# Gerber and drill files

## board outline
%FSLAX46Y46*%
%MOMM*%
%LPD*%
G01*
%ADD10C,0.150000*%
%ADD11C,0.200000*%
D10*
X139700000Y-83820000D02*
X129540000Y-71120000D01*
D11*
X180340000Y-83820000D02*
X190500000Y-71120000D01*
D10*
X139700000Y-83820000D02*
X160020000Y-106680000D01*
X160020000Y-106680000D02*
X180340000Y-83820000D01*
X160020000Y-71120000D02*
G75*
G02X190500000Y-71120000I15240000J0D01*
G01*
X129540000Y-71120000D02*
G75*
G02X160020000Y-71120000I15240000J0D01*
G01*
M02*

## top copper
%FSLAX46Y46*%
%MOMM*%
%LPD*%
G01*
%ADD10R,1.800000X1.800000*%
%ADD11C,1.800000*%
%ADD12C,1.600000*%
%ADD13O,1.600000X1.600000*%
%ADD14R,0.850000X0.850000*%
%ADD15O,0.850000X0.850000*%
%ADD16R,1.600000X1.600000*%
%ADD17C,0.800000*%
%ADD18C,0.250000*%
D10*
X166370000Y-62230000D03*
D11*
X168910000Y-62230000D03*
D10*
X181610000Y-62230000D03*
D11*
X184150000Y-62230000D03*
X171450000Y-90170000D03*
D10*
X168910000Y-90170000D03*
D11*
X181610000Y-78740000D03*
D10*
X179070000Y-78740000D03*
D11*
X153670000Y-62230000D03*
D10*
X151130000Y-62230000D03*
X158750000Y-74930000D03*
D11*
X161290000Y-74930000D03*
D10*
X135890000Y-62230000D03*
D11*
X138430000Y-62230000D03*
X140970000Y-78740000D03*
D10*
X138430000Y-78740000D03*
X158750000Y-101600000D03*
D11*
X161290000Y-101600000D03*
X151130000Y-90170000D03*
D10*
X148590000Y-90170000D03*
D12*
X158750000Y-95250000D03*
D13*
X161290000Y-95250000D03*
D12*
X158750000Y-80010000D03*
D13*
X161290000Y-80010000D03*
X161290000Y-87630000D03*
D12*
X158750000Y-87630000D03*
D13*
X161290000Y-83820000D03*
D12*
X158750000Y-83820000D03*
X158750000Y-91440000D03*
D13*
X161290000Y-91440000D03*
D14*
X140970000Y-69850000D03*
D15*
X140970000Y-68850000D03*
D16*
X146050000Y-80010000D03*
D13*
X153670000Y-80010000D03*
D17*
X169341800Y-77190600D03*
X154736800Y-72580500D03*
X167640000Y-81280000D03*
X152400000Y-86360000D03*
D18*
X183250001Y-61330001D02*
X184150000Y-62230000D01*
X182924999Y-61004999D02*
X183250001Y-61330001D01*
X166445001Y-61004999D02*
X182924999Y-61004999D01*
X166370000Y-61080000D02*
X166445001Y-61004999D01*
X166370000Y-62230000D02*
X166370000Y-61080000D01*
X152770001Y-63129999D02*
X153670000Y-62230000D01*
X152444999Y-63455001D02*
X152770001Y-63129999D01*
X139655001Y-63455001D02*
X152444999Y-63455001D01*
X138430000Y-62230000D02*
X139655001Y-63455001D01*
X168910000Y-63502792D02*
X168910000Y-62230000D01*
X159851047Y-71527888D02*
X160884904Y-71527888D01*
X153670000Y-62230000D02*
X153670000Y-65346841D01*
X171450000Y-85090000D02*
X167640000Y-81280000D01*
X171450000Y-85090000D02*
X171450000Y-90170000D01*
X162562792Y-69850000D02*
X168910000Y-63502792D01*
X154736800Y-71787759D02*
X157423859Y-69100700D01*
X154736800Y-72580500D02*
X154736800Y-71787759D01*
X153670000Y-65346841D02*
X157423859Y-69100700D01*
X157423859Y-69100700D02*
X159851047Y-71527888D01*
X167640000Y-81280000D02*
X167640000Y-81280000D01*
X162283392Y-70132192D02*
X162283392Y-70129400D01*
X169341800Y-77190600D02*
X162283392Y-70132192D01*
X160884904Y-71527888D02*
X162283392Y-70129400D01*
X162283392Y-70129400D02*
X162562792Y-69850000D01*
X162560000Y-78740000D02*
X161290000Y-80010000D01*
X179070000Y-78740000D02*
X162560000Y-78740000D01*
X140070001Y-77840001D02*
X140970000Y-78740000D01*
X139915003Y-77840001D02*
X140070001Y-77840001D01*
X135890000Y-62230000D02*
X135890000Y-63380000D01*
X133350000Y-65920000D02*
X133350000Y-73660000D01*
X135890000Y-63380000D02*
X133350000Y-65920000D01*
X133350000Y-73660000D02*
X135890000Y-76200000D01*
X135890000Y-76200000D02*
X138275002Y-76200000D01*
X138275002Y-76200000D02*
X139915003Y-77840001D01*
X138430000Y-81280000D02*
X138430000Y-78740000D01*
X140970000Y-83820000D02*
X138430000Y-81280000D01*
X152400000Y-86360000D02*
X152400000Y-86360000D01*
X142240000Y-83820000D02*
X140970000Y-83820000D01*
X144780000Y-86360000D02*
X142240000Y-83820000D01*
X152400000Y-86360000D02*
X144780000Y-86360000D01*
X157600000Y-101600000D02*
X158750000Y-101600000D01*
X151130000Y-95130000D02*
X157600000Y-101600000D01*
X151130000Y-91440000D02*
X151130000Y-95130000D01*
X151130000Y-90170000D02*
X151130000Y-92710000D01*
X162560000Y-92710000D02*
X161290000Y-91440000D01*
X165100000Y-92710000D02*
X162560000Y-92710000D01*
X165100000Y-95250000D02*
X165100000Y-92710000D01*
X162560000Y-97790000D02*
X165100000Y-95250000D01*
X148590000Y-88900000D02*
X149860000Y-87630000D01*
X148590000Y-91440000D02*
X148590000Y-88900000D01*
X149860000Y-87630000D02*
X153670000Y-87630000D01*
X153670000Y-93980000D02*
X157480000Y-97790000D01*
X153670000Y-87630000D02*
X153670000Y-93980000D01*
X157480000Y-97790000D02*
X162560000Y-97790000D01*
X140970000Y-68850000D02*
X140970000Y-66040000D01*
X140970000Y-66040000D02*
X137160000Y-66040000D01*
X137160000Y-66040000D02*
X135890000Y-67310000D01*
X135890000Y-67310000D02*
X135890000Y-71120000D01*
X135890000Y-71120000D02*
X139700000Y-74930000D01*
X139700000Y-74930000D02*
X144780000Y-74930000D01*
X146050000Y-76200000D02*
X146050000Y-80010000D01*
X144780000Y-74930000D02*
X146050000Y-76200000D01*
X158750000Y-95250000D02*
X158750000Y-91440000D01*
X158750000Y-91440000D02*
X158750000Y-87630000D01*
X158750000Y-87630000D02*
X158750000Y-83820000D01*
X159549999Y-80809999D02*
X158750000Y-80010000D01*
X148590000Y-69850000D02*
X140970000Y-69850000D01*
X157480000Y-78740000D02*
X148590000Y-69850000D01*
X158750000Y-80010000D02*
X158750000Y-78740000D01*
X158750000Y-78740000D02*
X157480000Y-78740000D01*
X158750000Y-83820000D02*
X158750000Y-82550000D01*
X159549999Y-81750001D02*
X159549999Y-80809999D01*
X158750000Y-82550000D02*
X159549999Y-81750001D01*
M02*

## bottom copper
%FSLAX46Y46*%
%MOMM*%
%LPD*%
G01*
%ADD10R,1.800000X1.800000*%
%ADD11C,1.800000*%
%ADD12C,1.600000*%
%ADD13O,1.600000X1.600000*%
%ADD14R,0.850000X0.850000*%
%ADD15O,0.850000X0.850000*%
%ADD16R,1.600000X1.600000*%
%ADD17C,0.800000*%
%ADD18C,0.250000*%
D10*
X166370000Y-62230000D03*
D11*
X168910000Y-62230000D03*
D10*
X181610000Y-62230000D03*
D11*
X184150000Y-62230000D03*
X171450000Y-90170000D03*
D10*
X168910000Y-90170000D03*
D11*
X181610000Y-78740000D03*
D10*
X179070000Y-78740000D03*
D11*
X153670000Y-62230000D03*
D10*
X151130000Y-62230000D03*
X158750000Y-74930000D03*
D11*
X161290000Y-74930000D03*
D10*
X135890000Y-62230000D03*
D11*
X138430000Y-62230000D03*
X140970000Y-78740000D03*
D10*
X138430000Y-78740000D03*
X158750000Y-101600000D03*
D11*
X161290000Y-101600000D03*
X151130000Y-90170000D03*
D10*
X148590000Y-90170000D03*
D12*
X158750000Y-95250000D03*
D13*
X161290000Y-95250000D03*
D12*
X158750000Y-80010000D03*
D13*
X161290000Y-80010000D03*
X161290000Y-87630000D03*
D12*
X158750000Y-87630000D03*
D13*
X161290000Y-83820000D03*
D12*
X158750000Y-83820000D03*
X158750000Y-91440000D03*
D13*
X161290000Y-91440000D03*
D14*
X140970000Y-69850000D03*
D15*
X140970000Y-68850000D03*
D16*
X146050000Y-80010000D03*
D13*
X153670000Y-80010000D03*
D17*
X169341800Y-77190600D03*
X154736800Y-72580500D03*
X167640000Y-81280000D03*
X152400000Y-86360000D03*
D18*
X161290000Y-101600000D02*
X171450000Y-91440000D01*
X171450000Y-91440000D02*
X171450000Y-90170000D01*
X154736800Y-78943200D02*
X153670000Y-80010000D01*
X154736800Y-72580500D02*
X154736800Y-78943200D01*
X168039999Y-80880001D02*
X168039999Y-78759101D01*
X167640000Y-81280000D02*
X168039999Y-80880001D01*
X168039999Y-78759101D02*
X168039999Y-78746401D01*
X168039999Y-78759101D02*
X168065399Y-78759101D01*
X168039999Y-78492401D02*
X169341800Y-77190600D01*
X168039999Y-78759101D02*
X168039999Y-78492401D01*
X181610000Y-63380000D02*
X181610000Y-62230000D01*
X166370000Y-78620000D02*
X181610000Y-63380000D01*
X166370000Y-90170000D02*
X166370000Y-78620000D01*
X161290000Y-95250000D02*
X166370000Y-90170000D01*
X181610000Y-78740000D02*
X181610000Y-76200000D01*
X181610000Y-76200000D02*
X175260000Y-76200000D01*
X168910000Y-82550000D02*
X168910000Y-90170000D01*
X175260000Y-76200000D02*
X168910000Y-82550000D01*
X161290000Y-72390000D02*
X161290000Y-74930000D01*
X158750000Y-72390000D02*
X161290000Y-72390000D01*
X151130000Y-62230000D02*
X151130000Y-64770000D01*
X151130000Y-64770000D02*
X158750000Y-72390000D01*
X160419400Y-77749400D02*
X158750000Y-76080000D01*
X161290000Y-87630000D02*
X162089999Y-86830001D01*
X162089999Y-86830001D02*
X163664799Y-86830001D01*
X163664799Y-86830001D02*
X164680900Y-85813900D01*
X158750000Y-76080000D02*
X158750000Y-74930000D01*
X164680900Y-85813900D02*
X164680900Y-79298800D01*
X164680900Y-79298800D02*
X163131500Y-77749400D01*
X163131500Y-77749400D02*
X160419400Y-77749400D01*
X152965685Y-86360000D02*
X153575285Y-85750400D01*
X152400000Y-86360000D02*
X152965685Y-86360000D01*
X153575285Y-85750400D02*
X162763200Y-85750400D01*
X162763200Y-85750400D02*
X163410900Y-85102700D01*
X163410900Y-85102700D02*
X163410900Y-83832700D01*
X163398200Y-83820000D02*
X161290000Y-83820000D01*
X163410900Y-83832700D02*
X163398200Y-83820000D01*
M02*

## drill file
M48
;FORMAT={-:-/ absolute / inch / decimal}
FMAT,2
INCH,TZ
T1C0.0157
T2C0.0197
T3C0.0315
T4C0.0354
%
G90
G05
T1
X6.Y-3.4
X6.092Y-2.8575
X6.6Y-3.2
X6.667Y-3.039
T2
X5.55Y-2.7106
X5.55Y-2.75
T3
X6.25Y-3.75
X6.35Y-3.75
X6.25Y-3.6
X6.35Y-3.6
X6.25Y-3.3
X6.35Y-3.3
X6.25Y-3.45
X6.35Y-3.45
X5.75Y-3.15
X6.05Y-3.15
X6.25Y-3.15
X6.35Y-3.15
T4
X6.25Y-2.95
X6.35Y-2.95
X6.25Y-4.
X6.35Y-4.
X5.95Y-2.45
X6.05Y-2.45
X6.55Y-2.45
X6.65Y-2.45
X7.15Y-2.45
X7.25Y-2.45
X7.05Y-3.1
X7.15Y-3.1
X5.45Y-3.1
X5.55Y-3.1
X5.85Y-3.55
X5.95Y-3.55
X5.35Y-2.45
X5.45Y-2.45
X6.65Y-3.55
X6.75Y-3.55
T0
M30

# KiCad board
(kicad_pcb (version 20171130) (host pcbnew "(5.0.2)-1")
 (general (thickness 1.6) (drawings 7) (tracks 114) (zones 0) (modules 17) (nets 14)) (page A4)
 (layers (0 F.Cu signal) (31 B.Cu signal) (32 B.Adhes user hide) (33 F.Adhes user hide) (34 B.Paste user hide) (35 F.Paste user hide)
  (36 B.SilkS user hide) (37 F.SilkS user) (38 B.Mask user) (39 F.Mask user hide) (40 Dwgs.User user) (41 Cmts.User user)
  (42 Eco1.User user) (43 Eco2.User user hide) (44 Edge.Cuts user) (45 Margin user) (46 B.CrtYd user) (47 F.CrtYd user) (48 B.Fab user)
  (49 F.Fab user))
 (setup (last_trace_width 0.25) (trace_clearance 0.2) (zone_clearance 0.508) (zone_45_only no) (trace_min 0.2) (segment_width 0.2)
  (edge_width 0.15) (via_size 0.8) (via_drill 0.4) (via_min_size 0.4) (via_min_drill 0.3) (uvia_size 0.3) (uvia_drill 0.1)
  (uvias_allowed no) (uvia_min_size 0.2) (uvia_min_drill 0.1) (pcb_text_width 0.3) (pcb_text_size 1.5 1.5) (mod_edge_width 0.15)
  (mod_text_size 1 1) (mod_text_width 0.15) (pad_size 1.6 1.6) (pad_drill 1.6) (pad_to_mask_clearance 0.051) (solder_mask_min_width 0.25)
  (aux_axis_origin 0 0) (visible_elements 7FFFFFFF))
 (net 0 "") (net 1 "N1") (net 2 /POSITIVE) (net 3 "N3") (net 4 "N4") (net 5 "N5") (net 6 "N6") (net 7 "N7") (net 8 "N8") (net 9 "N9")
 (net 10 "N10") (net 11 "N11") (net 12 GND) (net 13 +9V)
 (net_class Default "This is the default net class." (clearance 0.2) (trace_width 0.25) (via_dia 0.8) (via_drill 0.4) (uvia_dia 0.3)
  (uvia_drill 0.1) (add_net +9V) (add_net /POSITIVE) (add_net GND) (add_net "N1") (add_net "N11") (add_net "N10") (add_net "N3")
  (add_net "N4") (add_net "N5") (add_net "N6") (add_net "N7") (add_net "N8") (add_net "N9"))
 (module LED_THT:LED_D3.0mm (layer F.Cu) (at 166.37 62.23)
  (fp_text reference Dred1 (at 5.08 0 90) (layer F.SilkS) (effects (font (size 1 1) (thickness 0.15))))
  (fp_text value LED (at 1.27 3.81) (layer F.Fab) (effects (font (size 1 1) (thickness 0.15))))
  (pad 1 thru_hole rect (at 0 0) (size 1.8 1.8) (drill 0.9) (layers *.Cu *.Mask) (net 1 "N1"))
  (pad 2 thru_hole circle (at 2.54 0) (size 1.8 1.8) (drill 0.9) (layers *.Cu *.Mask) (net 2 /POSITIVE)))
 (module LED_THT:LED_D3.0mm (layer F.Cu) (at 181.61 62.23)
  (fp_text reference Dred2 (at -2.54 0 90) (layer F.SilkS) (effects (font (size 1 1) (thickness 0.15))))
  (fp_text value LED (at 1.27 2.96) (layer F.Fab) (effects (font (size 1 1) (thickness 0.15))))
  (pad 1 thru_hole rect (at 0 0) (size 1.8 1.8) (drill 0.9) (layers *.Cu *.Mask) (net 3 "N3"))
  (pad 2 thru_hole circle (at 2.54 0) (size 1.8 1.8) (drill 0.9) (layers *.Cu *.Mask) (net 1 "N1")))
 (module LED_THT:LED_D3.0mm (layer F.Cu) (at 168.91 90.17)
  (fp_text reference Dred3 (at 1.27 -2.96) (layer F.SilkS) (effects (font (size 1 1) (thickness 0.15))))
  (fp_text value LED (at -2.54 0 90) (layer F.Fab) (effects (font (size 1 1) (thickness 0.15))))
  (pad 2 thru_hole circle (at 2.54 0) (size 1.8 1.8) (drill 0.9) (layers *.Cu *.Mask) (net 2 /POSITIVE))
  (pad 1 thru_hole rect (at 0 0) (size 1.8 1.8) (drill 0.9) (layers *.Cu *.Mask) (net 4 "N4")))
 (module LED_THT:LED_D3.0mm (layer F.Cu) (at 179.07 78.74)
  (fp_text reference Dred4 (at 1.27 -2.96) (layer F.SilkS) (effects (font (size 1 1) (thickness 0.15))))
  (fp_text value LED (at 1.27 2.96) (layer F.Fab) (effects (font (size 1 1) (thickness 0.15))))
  (pad 2 thru_hole circle (at 2.54 0) (size 1.8 1.8) (drill 0.9) (layers *.Cu *.Mask) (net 4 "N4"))
  (pad 1 thru_hole rect (at 0 0) (size 1.8 1.8) (drill 0.9) (layers *.Cu *.Mask) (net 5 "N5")))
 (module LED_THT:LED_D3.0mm (layer F.Cu) (at 151.13 62.23)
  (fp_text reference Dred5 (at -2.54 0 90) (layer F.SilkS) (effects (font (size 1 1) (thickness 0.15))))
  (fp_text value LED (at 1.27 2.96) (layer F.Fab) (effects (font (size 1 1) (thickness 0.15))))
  (pad 2 thru_hole circle (at 2.54 0) (size 1.8 1.8) (drill 0.9) (layers *.Cu *.Mask) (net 2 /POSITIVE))
  (pad 1 thru_hole rect (at 0 0) (size 1.8 1.8) (drill 0.9) (layers *.Cu *.Mask) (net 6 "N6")))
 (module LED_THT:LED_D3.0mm (layer F.Cu) (at 158.75 74.93)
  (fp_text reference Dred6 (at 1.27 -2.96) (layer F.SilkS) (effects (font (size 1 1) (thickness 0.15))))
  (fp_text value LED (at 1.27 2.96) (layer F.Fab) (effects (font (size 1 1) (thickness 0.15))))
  (pad 1 thru_hole rect (at 0 0) (size 1.8 1.8) (drill 0.9) (layers *.Cu *.Mask) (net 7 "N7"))
  (pad 2 thru_hole circle (at 2.54 0) (size 1.8 1.8) (drill 0.9) (layers *.Cu *.Mask) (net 6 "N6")))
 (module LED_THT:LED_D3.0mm (layer F.Cu) (at 135.89 62.23)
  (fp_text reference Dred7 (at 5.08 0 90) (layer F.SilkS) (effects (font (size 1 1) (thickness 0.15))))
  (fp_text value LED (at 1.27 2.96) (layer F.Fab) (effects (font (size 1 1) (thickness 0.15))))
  (pad 1 thru_hole rect (at 0 0) (size 1.8 1.8) (drill 0.9) (layers *.Cu *.Mask) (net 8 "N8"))
  (pad 2 thru_hole circle (at 2.54 0) (size 1.8 1.8) (drill 0.9) (layers *.Cu *.Mask) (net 2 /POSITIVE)))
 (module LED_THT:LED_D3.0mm (layer F.Cu) (at 138.43 78.74)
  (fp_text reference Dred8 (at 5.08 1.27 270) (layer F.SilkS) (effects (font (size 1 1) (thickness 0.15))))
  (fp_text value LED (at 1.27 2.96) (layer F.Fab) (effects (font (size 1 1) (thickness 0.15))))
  (pad 2 thru_hole circle (at 2.54 0) (size 1.8 1.8) (drill 0.9) (layers *.Cu *.Mask) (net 8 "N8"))
  (pad 1 thru_hole rect (at 0 0) (size 1.8 1.8) (drill 0.9) (layers *.Cu *.Mask) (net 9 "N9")))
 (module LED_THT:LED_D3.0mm (layer F.Cu) (at 158.75 101.6)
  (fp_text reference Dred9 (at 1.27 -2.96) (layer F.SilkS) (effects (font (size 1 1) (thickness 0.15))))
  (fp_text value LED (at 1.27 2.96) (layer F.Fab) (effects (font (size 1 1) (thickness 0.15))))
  (pad 1 thru_hole rect (at 0 0) (size 1.8 1.8) (drill 0.9) (layers *.Cu *.Mask) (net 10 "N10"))
  (pad 2 thru_hole circle (at 2.54 0) (size 1.8 1.8) (drill 0.9) (layers *.Cu *.Mask) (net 2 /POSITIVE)))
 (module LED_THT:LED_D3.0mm (layer F.Cu) (at 148.59 90.17)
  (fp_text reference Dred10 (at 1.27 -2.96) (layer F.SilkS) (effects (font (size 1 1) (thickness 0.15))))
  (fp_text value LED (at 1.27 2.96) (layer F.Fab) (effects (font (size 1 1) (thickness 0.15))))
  (pad 2 thru_hole circle (at 2.54 0) (size 1.8 1.8) (drill 0.9) (layers *.Cu *.Mask) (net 10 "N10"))
  (pad 1 thru_hole rect (at 0 0) (size 1.8 1.8) (drill 0.9) (layers *.Cu *.Mask) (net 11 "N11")))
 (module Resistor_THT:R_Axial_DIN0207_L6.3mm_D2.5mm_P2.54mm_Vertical (layer F.Cu) (at 158.75 95.25)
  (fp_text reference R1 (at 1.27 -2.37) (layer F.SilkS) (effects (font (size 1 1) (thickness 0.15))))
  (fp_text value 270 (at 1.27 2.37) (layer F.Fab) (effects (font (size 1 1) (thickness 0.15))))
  (pad 1 thru_hole circle (at 0 0) (size 1.6 1.6) (drill 0.8) (layers *.Cu *.Mask) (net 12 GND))
  (pad 2 thru_hole oval (at 2.54 0) (size 1.6 1.6) (drill 0.8) (layers *.Cu *.Mask) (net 3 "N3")))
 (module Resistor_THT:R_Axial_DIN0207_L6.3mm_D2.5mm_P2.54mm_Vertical (layer F.Cu) (at 158.75 80.01)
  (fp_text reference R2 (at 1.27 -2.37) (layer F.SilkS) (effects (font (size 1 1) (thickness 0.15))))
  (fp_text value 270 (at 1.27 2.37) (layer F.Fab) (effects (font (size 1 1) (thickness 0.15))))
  (pad 1 thru_hole circle (at 0 0) (size 1.6 1.6) (drill 0.8) (layers *.Cu *.Mask) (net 12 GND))
  (pad 2 thru_hole oval (at 2.54 0) (size 1.6 1.6) (drill 0.8) (layers *.Cu *.Mask) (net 5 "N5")))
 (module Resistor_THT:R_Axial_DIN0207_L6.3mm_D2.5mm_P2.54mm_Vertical (layer F.Cu) (at 158.75 87.63)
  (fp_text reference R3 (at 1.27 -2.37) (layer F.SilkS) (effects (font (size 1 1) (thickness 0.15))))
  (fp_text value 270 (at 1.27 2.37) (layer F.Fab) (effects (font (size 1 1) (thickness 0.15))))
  (pad 2 thru_hole oval (at 2.54 0) (size 1.6 1.6) (drill 0.8) (layers *.Cu *.Mask) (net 7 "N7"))
  (pad 1 thru_hole circle (at 0 0) (size 1.6 1.6) (drill 0.8) (layers *.Cu *.Mask) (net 12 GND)))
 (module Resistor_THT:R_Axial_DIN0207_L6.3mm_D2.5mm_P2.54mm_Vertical (layer F.Cu) (at 158.75 83.82)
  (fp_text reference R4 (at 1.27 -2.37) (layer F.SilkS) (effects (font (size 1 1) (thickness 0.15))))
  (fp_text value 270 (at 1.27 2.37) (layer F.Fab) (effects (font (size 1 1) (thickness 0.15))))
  (pad 2 thru_hole oval (at 2.54 0) (size 1.6 1.6) (drill 0.8) (layers *.Cu *.Mask) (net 9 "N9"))
  (pad 1 thru_hole circle (at 0 0) (size 1.6 1.6) (drill 0.8) (layers *.Cu *.Mask) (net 12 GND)))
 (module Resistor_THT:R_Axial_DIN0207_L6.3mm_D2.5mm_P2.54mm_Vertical (layer F.Cu) (at 158.75 91.44)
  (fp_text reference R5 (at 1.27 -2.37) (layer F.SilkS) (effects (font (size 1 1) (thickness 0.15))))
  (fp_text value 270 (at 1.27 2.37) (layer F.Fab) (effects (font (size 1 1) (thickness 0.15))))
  (pad 1 thru_hole circle (at 0 0) (size 1.6 1.6) (drill 0.8) (layers *.Cu *.Mask) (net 12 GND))
  (pad 2 thru_hole oval (at 2.54 0) (size 1.6 1.6) (drill 0.8) (layers *.Cu *.Mask) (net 11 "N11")))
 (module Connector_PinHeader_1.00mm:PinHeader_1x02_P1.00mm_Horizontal (layer F.Cu) (at 140.97 69.85 180)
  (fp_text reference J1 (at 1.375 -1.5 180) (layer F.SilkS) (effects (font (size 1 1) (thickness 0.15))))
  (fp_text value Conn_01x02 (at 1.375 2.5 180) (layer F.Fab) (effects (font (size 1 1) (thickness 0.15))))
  (pad 1 thru_hole rect (at 0 0 180) (size 0.85 0.85) (drill 0.5) (layers *.Cu *.Mask) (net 12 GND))
  (pad 2 thru_hole oval (at 0 1 180) (size 0.85 0.85) (drill 0.5) (layers *.Cu *.Mask) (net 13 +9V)))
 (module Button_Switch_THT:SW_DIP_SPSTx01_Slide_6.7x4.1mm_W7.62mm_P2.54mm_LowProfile (layer F.Cu) (at 146.05 80.01)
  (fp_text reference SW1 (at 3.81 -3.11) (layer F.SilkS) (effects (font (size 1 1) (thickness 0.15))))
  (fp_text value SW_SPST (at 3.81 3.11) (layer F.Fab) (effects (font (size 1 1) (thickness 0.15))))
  (pad 1 thru_hole rect (at 0 0) (size 1.6 1.6) (drill 0.8) (layers *.Cu *.Mask) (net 13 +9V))
  (pad 2 thru_hole oval (at 7.62 0) (size 1.6 1.6) (drill 0.8) (layers *.Cu *.Mask) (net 2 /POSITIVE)))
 (gr_line (start 139.7 83.82) (end 129.54 71.12) (layer Edge.Cuts) (width 0.15))
 (gr_line (start 180.34 83.82) (end 190.5 71.12) (layer Edge.Cuts) (width 0.2))
 (gr_line (start 139.7 83.82) (end 160.02 106.68) (layer Edge.Cuts) (width 0.15))
 (gr_line (start 160.02 106.68) (end 180.34 83.82) (layer Edge.Cuts) (width 0.15))
 (gr_arc (start 175.26 71.12) (end 190.5 71.12) (angle -180) (layer Edge.Cuts) (width 0.15))
 (gr_arc (start 144.78 71.12) (end 160.02 71.12) (angle -180) (layer Edge.Cuts) (width 0.15))
 (segment (start 183.250001 61.330001) (end 184.15 62.23) (width 0.25) (layer F.Cu) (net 1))
 (segment (start 182.924999 61.004999) (end 183.250001 61.330001) (width 0.25) (layer F.Cu) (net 1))
 (segment (start 166.445001 61.004999) (end 182.924999 61.004999) (width 0.25) (layer F.Cu) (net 1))
 (segment (start 166.37 61.08) (end 166.445001 61.004999) (width 0.25) (layer F.Cu) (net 1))
 (segment (start 166.37 62.23) (end 166.37 61.08) (width 0.25) (layer F.Cu) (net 1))
 (via (at 169.3418 77.1906) (size 0.8) (drill 0.4) (layers F.Cu B.Cu) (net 2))
 (via (at 154.7368 72.5805) (size 0.8) (drill 0.4) (layers F.Cu B.Cu) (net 2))
 (segment (start 161.29 101.6) (end 171.45 91.44) (width 0.25) (layer B.Cu) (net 2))
 (segment (start 152.770001 63.129999) (end 153.67 62.23) (width 0.25) (layer F.Cu) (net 2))
 (segment (start 152.444999 63.455001) (end 152.770001 63.129999) (width 0.25) (layer F.Cu) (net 2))
 (segment (start 139.655001 63.455001) (end 152.444999 63.455001) (width 0.25) (layer F.Cu) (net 2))
 (segment (start 138.43 62.23) (end 139.655001 63.455001) (width 0.25) (layer F.Cu) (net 2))
 (segment (start 168.91 63.502792) (end 168.91 62.23) (width 0.25) (layer F.Cu) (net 2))
 (segment (start 159.851047 71.527888) (end 160.884904 71.527888) (width 0.25) (layer F.Cu) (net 2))
 (segment (start 153.67 62.23) (end 153.67 65.346841) (width 0.25) (layer F.Cu) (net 2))
 (segment (start 171.45 85.09) (end 167.64 81.28) (width 0.25) (layer F.Cu) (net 2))
 (segment (start 171.45 85.09) (end 171.45 90.17) (width 0.25) (layer F.Cu) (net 2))
 (segment (start 171.45 91.44) (end 171.45 90.17) (width 0.25) (layer B.Cu) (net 2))
 (segment (start 162.562792 69.85) (end 168.91 63.502792) (width 0.25) (layer F.Cu) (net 2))
 (segment (start 154.7368 71.787759) (end 157.423859 69.1007) (width 0.25) (layer F.Cu) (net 2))
 (segment (start 154.7368 72.5805) (end 154.7368 71.787759) (width 0.25) (layer F.Cu) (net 2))
 (segment (start 153.67 65.346841) (end 157.423859 69.1007) (width 0.25) (layer F.Cu) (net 2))
 (segment (start 157.423859 69.1007) (end 159.851047 71.527888) (width 0.25) (layer F.Cu) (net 2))
 (segment (start 154.7368 78.9432) (end 153.67 80.01) (width 0.25) (layer B.Cu) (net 2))
 (segment (start 154.7368 72.5805) (end 154.7368 78.9432) (width 0.25) (layer B.Cu) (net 2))
 (segment (start 167.64 81.28) (end 167.64 81.28) (width 0.25) (layer F.Cu) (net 2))
 (via (at 167.64 81.28) (size 0.8) (drill 0.4) (layers F.Cu B.Cu) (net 2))
 (segment (start 168.039999 80.880001) (end 168.039999 78.759101) (width 0.25) (layer B.Cu) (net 2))
 (segment (start 167.64 81.28) (end 168.039999 80.880001) (width 0.25) (layer B.Cu) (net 2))
 (segment (start 168.039999 78.759101) (end 168.039999 78.746401) (width 0.25) (layer B.Cu) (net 2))
 (segment (start 168.039999 78.759101) (end 168.065399 78.759101) (width 0.25) (layer B.Cu) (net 2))
 (segment (start 168.039999 78.492401) (end 169.3418 77.1906) (width 0.25) (layer B.Cu) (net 2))
 (segment (start 168.039999 78.759101) (end 168.039999 78.492401) (width 0.25) (layer B.Cu) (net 2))
 (segment (start 162.283392 70.132192) (end 162.283392 70.1294) (width 0.25) (layer F.Cu) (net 2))
 (segment (start 169.3418 77.1906) (end 162.283392 70.132192) (width 0.25) (layer F.Cu) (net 2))
 (segment (start 160.884904 71.527888) (end 162.283392 70.1294) (width 0.25) (layer F.Cu) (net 2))
 (segment (start 162.283392 70.1294) (end 162.562792 69.85) (width 0.25) (layer F.Cu) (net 2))
 (segment (start 181.61 63.38) (end 181.61 62.23) (width 0.25) (layer B.Cu) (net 3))
 (segment (start 166.37 78.62) (end 181.61 63.38) (width 0.25) (layer B.Cu) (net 3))
 (segment (start 166.37 90.17) (end 166.37 78.62) (width 0.25) (layer B.Cu) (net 3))
 (segment (start 161.29 95.25) (end 166.37 90.17) (width 0.25) (layer B.Cu) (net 3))
 (segment (start 181.61 78.74) (end 181.61 76.2) (width 0.25) (layer B.Cu) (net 4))
 (segment (start 181.61 76.2) (end 175.26 76.2) (width 0.25) (layer B.Cu) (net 4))
 (segment (start 168.91 82.55) (end 168.91 90.17) (width 0.25) (layer B.Cu) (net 4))
 (segment (start 175.26 76.2) (end 168.91 82.55) (width 0.25) (layer B.Cu) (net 4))
 (segment (start 162.56 78.74) (end 161.29 80.01) (width 0.25) (layer F.Cu) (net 5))
 (segment (start 179.07 78.74) (end 162.56 78.74) (width 0.25) (layer F.Cu) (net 5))
 (segment (start 161.29 72.39) (end 161.29 74.93) (width 0.25) (layer B.Cu) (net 6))
 (segment (start 158.75 72.39) (end 161.29 72.39) (width 0.25) (layer B.Cu) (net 6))
 (segment (start 151.13 62.23) (end 151.13 64.77) (width 0.25) (layer B.Cu) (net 6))
 (segment (start 151.13 64.77) (end 158.75 72.39) (width 0.25) (layer B.Cu) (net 6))
 (segment (start 160.4194 77.7494) (end 158.75 76.08) (width 0.25) (layer B.Cu) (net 7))
 (segment (start 161.29 87.63) (end 162.089999 86.830001) (width 0.25) (layer B.Cu) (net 7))
 (segment (start 162.089999 86.830001) (end 163.664799 86.830001) (width 0.25) (layer B.Cu) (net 7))
 (segment (start 163.664799 86.830001) (end 164.6809 85.8139) (width 0.25) (layer B.Cu) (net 7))
 (segment (start 158.75 76.08) (end 158.75 74.93) (width 0.25) (layer B.Cu) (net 7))
 (segment (start 164.6809 85.8139) (end 164.6809 79.2988) (width 0.25) (layer B.Cu) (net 7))
 (segment (start 164.6809 79.2988) (end 163.1315 77.7494) (width 0.25) (layer B.Cu) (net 7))
 (segment (start 163.1315 77.7494) (end 160.4194 77.7494) (width 0.25) (layer B.Cu) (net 7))
 (segment (start 140.070001 77.840001) (end 140.97 78.74) (width 0.25) (layer F.Cu) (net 8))
 (segment (start 139.915003 77.840001) (end 140.070001 77.840001) (width 0.25) (layer F.Cu) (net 8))
 (segment (start 135.89 62.23) (end 135.89 63.38) (width 0.25) (layer F.Cu) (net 8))
 (segment (start 133.35 65.92) (end 133.35 73.66) (width 0.25) (layer F.Cu) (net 8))
 (segment (start 135.89 63.38) (end 133.35 65.92) (width 0.25) (layer F.Cu) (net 8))
 (segment (start 133.35 73.66) (end 135.89 76.2) (width 0.25) (layer F.Cu) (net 8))
 (segment (start 135.89 76.2) (end 138.275002 76.2) (width 0.25) (layer F.Cu) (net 8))
 (segment (start 138.275002 76.2) (end 139.915003 77.840001) (width 0.25) (layer F.Cu) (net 8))
 (segment (start 138.43 81.28) (end 138.43 78.74) (width 0.25) (layer F.Cu) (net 9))
 (segment (start 140.97 83.82) (end 138.43 81.28) (width 0.25) (layer F.Cu) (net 9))
 (segment (start 152.4 86.36) (end 152.4 86.36) (width 0.25) (layer F.Cu) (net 9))
 (segment (start 142.24 83.82) (end 140.97 83.82) (width 0.25) (layer F.Cu) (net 9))
 (segment (start 144.78 86.36) (end 142.24 83.82) (width 0.25) (layer F.Cu) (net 9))
 (segment (start 152.4 86.36) (end 144.78 86.36) (width 0.25) (layer F.Cu) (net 9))
 (via (at 152.4 86.36) (size 0.8) (drill 0.4) (layers F.Cu B.Cu) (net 9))
 (segment (start 152.965685 86.36) (end 153.575285 85.7504) (width 0.25) (layer B.Cu) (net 9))
 (segment (start 152.4 86.36) (end 152.965685 86.36) (width 0.25) (layer B.Cu) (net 9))
 (segment (start 153.575285 85.7504) (end 162.7632 85.7504) (width 0.25) (layer B.Cu) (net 9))
 (segment (start 162.7632 85.7504) (end 163.4109 85.1027) (width 0.25) (layer B.Cu) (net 9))
 (segment (start 163.4109 85.1027) (end 163.4109 83.8327) (width 0.25) (layer B.Cu) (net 9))
 (segment (start 163.3982 83.82) (end 161.29 83.82) (width 0.25) (layer B.Cu) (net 9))
 (segment (start 163.4109 83.8327) (end 163.3982 83.82) (width 0.25) (layer B.Cu) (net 9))
 (segment (start 157.6 101.6) (end 158.75 101.6) (width 0.25) (layer F.Cu) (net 10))
 (segment (start 151.13 95.13) (end 157.6 101.6) (width 0.25) (layer F.Cu) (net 10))
 (segment (start 151.13 91.44) (end 151.13 95.13) (width 0.25) (layer F.Cu) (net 10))
 (segment (start 151.13 90.17) (end 151.13 92.71) (width 0.25) (layer F.Cu) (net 10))
 (segment (start 162.56 92.71) (end 161.29 91.44) (width 0.25) (layer F.Cu) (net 11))
 (segment (start 165.1 92.71) (end 162.56 92.71) (width 0.25) (layer F.Cu) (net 11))
 (segment (start 165.1 95.25) (end 165.1 92.71) (width 0.25) (layer F.Cu) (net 11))
 (segment (start 162.56 97.79) (end 165.1 95.25) (width 0.25) (layer F.Cu) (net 11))
 (segment (start 148.59 88.9) (end 149.86 87.63) (width 0.25) (layer F.Cu) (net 11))
 (segment (start 148.59 91.44) (end 148.59 88.9) (width 0.25) (layer F.Cu) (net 11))
 (segment (start 149.86 87.63) (end 153.67 87.63) (width 0.25) (layer F.Cu) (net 11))
 (segment (start 153.67 93.98) (end 157.48 97.79) (width 0.25) (layer F.Cu) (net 11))
 (segment (start 153.67 87.63) (end 153.67 93.98) (width 0.25) (layer F.Cu) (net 11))
 (segment (start 157.48 97.79) (end 162.56 97.79) (width 0.25) (layer F.Cu) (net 11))
 (segment (start 140.97 68.85) (end 140.97 66.04) (width 0.25) (layer F.Cu) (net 13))
 (segment (start 140.97 66.04) (end 137.16 66.04) (width 0.25) (layer F.Cu) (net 13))
 (segment (start 137.16 66.04) (end 135.89 67.31) (width 0.25) (layer F.Cu) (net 13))
 (segment (start 135.89 67.31) (end 135.89 71.12) (width 0.25) (layer F.Cu) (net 13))
 (segment (start 135.89 71.12) (end 139.7 74.93) (width 0.25) (layer F.Cu) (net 13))
 (segment (start 139.7 74.93) (end 144.78 74.93) (width 0.25) (layer F.Cu) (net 13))
 (segment (start 146.05 76.2) (end 146.05 80.01) (width 0.25) (layer F.Cu) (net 13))
 (segment (start 144.78 74.93) (end 146.05 76.2) (width 0.25) (layer F.Cu) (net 13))
 (segment (start 158.75 95.25) (end 158.75 91.44) (width 0.25) (layer F.Cu) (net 12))
 (segment (start 158.75 91.44) (end 158.75 87.63) (width 0.25) (layer F.Cu) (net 12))
 (segment (start 158.75 87.63) (end 158.75 83.82) (width 0.25) (layer F.Cu) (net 12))
 (segment (start 159.549999 80.809999) (end 158.75 80.01) (width 0.25) (layer F.Cu) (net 12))
 (segment (start 148.59 69.85) (end 140.97 69.85) (width 0.25) (layer F.Cu) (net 12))
 (segment (start 157.48 78.74) (end 148.59 69.85) (width 0.25) (layer F.Cu) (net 12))
 (segment (start 158.75 80.01) (end 158.75 78.74) (width 0.25) (layer F.Cu) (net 12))
 (segment (start 158.75 78.74) (end 157.48 78.74) (width 0.25) (layer F.Cu) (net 12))
 (segment (start 158.75 83.82) (end 158.75 82.55) (width 0.25) (layer F.Cu) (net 12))
 (segment (start 159.549999 81.750001) (end 159.549999 80.809999) (width 0.25) (layer F.Cu) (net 12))
 (segment (start 158.75 82.55) (end 159.549999 81.750001) (width 0.25) (layer F.Cu) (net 12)))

